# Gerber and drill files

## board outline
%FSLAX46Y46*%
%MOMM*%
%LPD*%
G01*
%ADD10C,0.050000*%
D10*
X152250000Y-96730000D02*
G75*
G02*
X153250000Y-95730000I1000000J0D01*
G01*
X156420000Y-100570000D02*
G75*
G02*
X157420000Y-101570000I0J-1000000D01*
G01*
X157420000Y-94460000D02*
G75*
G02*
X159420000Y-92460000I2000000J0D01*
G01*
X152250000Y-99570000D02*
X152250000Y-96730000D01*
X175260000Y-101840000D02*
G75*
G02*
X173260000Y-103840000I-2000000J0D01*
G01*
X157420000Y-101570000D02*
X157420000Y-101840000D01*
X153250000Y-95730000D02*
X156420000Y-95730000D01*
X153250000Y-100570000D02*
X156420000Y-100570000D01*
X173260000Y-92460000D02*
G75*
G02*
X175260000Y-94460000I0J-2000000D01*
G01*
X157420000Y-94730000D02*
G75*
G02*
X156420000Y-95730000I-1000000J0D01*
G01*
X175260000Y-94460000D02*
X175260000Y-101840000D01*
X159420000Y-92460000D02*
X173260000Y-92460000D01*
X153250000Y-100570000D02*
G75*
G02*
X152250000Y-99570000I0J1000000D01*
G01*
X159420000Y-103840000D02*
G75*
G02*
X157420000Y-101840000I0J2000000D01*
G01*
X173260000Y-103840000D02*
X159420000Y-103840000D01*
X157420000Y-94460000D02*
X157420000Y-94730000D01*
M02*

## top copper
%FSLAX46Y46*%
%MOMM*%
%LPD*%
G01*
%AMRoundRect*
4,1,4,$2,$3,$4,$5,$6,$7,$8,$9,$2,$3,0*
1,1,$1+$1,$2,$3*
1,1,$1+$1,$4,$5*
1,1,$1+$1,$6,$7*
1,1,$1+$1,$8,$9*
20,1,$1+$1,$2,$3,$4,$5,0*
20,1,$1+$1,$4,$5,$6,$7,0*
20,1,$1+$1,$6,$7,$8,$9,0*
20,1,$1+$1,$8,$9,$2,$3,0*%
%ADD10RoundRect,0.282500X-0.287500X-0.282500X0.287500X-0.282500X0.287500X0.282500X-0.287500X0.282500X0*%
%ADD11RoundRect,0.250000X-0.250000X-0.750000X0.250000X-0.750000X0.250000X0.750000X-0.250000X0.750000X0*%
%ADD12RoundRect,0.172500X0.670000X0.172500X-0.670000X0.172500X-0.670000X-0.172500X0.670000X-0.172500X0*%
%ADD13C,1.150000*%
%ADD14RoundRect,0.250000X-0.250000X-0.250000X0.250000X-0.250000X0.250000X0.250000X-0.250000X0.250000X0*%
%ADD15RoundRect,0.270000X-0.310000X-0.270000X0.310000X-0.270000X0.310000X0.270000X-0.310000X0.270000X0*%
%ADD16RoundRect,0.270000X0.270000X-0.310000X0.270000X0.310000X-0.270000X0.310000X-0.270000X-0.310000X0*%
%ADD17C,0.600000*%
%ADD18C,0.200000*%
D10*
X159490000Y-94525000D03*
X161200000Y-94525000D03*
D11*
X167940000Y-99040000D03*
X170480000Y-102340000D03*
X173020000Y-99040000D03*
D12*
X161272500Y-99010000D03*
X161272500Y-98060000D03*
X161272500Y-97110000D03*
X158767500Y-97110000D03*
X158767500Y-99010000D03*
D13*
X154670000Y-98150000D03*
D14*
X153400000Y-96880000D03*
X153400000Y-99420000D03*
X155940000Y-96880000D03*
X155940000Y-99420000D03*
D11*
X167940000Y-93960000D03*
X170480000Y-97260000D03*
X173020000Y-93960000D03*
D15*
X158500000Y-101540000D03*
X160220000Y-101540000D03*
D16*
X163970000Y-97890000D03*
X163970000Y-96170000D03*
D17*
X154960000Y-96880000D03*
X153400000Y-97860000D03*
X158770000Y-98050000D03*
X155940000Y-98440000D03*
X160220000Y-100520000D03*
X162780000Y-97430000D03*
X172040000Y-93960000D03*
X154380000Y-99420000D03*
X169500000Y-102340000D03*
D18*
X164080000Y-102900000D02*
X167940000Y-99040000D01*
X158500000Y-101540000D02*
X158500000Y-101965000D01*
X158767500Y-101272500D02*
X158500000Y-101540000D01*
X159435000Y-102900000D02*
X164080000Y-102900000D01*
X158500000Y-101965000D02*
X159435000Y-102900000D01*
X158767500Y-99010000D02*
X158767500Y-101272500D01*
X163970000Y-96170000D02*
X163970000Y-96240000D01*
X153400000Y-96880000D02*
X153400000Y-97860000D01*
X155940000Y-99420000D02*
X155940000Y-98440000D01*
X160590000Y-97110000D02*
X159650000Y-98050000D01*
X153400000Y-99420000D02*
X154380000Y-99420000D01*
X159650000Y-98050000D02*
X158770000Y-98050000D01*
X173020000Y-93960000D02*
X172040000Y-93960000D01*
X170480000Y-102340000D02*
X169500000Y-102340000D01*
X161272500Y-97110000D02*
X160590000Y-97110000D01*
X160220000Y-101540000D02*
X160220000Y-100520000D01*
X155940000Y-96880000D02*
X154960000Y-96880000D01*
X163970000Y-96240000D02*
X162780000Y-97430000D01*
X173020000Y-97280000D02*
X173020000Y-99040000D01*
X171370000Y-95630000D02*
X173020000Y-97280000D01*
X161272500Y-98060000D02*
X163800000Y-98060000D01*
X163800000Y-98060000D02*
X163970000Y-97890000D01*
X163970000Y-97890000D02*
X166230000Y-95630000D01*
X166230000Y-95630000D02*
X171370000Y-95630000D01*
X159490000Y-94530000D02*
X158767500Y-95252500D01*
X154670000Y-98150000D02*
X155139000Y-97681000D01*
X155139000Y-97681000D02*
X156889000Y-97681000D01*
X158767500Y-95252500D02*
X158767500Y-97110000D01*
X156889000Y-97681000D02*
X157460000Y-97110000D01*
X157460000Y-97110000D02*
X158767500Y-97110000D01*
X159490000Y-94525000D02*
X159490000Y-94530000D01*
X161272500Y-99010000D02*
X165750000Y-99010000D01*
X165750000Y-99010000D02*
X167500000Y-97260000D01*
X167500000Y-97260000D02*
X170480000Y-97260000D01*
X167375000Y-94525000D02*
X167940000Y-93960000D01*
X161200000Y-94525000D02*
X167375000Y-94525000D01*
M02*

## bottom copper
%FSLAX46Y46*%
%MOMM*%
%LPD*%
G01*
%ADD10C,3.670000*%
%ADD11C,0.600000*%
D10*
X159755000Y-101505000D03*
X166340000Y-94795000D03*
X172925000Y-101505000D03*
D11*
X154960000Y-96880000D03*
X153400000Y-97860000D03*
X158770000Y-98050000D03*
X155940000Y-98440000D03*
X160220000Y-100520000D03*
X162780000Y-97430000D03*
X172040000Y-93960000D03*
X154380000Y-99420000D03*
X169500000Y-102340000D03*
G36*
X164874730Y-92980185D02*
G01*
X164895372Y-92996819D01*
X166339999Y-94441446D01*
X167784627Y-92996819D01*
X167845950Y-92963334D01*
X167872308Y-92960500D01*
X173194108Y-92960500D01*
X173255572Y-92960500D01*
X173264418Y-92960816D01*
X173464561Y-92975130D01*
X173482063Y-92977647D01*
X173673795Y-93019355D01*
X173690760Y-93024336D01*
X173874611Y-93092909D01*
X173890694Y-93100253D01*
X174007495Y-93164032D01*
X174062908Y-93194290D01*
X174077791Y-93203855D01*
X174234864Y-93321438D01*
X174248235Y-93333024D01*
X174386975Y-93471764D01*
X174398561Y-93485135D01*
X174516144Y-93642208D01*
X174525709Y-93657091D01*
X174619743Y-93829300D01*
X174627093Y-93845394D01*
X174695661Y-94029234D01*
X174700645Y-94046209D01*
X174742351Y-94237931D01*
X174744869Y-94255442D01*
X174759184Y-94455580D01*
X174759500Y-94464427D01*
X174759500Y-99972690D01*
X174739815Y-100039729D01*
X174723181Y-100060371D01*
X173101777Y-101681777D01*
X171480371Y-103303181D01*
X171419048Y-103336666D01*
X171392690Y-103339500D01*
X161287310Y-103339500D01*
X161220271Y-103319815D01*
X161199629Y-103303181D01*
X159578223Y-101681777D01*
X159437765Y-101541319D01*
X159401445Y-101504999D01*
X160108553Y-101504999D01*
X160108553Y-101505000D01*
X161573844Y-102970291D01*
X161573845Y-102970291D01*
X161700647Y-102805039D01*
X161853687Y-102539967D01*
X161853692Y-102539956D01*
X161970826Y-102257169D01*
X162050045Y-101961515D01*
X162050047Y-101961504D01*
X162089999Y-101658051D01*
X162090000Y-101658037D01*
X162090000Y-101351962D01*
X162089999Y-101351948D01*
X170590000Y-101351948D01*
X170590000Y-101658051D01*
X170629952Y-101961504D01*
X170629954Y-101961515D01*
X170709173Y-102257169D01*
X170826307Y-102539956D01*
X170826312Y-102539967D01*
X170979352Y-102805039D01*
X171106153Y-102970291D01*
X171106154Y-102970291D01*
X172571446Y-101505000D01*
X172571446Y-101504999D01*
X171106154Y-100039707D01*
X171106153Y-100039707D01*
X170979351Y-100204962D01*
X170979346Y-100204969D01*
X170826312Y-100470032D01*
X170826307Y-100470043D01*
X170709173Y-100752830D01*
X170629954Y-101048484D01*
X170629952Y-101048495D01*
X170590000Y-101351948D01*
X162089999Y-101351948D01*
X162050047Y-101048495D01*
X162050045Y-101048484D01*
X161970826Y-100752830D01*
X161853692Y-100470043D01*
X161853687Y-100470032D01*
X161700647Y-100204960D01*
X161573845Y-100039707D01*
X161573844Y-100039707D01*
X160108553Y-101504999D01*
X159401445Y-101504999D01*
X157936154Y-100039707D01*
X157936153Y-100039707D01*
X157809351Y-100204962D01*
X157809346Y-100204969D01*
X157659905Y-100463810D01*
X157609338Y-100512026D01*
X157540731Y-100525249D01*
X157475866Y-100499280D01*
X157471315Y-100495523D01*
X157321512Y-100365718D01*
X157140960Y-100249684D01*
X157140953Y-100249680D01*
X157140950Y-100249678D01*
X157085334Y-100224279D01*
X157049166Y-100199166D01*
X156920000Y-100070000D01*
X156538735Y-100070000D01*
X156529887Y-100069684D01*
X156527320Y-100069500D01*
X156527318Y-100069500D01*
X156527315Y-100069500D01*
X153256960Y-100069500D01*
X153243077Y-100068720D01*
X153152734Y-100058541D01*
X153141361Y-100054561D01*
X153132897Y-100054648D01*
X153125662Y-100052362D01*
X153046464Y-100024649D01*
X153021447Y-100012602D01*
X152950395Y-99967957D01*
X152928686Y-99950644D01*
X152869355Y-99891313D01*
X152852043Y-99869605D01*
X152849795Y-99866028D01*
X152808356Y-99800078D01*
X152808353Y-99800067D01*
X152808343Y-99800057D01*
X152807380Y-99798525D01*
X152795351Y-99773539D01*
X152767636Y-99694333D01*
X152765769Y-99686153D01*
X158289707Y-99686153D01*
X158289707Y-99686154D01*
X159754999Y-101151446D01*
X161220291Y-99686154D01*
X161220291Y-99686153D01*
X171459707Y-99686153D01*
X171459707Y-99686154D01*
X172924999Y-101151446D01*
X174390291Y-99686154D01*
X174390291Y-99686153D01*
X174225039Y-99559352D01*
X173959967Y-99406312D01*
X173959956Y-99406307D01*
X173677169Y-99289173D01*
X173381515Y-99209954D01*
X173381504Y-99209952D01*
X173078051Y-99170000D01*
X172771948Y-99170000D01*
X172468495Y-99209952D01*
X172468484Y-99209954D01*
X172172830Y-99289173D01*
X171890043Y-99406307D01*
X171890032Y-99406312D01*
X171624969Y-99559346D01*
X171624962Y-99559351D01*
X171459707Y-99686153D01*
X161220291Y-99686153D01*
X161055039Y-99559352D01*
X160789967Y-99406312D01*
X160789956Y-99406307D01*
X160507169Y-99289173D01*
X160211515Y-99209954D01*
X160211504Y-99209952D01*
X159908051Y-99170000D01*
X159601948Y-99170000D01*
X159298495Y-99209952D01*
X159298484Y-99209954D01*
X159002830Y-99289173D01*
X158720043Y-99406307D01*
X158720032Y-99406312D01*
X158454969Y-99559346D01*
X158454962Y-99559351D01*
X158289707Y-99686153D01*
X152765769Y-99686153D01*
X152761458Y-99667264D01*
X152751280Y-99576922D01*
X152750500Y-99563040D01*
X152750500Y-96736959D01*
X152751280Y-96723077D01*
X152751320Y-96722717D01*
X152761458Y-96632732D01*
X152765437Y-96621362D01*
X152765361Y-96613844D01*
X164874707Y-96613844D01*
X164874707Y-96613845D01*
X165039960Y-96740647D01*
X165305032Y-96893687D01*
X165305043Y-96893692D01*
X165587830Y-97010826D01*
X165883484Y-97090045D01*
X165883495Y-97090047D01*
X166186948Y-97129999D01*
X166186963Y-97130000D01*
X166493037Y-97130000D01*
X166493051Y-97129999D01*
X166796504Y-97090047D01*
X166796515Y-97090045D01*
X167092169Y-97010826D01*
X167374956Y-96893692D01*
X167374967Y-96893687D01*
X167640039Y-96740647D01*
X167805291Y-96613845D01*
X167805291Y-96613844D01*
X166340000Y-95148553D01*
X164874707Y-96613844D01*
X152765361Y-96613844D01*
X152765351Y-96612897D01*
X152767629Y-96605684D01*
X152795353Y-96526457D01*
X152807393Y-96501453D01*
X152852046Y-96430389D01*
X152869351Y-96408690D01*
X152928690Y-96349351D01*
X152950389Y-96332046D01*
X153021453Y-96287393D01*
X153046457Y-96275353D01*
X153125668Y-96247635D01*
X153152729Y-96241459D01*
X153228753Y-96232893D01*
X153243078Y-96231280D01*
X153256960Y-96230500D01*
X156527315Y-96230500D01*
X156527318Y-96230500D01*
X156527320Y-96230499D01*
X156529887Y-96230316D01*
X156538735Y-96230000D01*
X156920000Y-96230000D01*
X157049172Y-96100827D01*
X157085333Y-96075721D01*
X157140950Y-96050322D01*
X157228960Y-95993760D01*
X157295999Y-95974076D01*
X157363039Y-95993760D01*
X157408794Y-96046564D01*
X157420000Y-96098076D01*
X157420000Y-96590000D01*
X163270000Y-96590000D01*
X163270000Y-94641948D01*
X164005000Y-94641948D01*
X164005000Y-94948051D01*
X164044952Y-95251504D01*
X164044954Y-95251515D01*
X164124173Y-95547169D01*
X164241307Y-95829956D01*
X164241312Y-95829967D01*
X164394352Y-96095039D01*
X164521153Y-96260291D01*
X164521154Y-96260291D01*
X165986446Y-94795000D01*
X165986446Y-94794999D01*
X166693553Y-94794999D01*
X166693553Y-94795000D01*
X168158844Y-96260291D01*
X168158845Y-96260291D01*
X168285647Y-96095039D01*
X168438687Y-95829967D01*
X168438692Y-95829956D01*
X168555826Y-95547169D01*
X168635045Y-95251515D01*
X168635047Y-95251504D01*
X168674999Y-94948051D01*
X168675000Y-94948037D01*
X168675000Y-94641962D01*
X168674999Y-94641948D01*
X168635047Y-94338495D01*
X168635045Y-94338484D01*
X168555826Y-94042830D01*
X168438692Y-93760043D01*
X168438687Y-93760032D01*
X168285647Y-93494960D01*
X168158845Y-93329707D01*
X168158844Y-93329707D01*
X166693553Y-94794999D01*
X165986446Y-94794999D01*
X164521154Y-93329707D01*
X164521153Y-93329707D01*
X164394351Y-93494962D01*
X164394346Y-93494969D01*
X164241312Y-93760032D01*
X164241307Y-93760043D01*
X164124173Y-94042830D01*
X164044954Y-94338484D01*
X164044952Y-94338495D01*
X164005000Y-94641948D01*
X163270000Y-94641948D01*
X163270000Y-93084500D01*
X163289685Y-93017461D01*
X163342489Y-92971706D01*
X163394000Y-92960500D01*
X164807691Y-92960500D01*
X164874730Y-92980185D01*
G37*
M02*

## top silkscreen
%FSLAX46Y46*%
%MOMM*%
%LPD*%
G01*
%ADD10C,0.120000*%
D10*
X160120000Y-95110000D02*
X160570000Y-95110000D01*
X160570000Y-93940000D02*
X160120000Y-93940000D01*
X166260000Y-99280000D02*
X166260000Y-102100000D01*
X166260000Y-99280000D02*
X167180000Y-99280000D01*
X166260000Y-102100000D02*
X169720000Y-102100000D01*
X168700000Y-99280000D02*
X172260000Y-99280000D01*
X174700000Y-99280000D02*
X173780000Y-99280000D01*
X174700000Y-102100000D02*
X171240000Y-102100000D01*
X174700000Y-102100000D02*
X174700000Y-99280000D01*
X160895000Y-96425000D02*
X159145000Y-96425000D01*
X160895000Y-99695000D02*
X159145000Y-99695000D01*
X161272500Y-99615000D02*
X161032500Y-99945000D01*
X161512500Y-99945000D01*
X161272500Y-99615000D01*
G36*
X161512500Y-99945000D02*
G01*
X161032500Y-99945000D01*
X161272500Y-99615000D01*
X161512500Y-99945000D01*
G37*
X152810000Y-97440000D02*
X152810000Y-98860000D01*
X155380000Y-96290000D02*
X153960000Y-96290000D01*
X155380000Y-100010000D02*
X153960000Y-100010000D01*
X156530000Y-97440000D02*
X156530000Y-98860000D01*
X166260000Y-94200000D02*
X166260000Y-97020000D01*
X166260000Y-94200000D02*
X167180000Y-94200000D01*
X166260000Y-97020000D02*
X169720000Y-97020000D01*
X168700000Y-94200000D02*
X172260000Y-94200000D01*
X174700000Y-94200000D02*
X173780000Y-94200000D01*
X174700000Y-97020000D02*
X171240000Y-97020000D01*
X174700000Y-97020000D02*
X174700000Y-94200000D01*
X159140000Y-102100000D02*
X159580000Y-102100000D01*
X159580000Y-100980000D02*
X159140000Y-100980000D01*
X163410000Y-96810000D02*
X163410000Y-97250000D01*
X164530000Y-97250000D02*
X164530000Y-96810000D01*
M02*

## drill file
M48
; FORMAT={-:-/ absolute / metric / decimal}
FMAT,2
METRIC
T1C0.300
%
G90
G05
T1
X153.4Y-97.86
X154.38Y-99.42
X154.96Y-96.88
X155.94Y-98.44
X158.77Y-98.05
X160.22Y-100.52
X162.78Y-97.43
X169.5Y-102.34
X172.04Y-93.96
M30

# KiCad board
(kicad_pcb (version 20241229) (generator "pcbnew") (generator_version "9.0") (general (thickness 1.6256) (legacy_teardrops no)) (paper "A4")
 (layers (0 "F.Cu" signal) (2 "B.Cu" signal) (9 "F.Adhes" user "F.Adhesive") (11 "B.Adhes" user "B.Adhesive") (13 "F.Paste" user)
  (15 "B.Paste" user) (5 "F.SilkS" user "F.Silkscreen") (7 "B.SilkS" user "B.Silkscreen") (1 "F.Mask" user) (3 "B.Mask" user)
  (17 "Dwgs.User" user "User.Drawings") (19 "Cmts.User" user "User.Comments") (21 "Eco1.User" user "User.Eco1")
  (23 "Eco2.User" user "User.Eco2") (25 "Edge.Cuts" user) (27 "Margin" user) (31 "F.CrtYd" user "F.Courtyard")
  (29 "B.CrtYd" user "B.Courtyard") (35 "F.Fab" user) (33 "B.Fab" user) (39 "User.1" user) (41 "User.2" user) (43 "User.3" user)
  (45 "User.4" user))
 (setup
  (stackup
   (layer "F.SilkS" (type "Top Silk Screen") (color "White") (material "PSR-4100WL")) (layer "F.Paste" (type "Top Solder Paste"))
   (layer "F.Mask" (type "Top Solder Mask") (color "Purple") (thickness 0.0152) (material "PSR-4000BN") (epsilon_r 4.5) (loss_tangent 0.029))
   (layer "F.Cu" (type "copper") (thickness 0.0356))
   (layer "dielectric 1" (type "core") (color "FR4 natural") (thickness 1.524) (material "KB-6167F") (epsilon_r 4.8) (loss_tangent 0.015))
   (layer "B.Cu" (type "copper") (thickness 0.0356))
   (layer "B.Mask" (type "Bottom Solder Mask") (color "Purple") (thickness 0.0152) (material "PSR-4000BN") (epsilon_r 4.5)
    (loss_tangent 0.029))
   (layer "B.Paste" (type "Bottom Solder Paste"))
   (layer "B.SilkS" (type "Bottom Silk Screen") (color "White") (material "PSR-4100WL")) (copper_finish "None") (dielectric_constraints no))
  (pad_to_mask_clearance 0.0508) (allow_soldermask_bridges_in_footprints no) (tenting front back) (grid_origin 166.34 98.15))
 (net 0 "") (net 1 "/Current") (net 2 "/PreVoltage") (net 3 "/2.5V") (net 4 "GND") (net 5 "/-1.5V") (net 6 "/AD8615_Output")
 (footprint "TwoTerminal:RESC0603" (layer "F.Cu") (at 160.345 94.525)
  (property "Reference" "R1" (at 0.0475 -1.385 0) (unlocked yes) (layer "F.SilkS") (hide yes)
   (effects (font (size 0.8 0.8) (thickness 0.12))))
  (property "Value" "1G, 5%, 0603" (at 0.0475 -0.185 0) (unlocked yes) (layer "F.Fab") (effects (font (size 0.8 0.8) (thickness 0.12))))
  (fp_line (start -0.225 0.585) (end 0.225 0.585) (stroke (width 0.12) (type default)) (layer "F.SilkS"))
  (fp_line (start 0.225 -0.585) (end -0.225 -0.585) (stroke (width 0.12) (type default)) (layer "F.SilkS"))
  (pad "1" smd roundrect (at -0.855 0) (size 1.14 1.13) (layers "F.Cu" "F.Mask" "F.Paste") (roundrect_rratio 0.25) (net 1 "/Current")
   (thermal_bridge_angle 45))
  (pad "2" smd roundrect (at 0.855 0) (size 1.14 1.13) (layers "F.Cu" "F.Mask" "F.Paste") (roundrect_rratio 0.25) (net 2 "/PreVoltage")
   (thermal_bridge_angle 45)))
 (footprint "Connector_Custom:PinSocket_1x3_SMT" (layer "F.Cu") (at 170.48 100.69 90)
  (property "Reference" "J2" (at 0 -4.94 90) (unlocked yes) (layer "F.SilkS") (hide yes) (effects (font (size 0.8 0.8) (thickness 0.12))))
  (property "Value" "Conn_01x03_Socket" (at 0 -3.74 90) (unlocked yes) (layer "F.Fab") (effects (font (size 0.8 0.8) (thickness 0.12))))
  (fp_line (start 1.41 -4.22) (end -1.41 -4.22) (stroke (width 0.12) (type default)) (layer "F.SilkS"))
  (fp_line (start 1.41 -4.22) (end 1.41 -3.3) (stroke (width 0.12) (type default)) (layer "F.SilkS"))
  (fp_line (start -1.41 -4.22) (end -1.41 -0.76) (stroke (width 0.12) (type default)) (layer "F.SilkS"))
  (fp_line (start 1.41 -1.78) (end 1.41 1.78) (stroke (width 0.12) (type default)) (layer "F.SilkS"))
  (fp_line (start 1.41 4.22) (end 1.41 3.3) (stroke (width 0.12) (type default)) (layer "F.SilkS"))
  (fp_line (start -1.41 4.22) (end -1.41 0.76) (stroke (width 0.12) (type default)) (layer "F.SilkS"))
  (fp_line (start -1.41 4.22) (end 1.41 4.22) (stroke (width 0.12) (type default)) (layer "F.SilkS"))
  (pad "1" smd roundrect (at 1.65 -2.54) (size 1 2) (layers "F.Cu" "F.Mask" "F.Paste") (roundrect_rratio 0.25) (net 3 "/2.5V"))
  (pad "2" smd roundrect (at -1.65 0) (size 1 2) (layers "F.Cu" "F.Mask" "F.Paste") (roundrect_rratio 0.25) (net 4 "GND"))
  (pad "3" smd roundrect (at 1.65 2.54) (size 1 2) (layers "F.Cu" "F.Mask" "F.Paste") (roundrect_rratio 0.25) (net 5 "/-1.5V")))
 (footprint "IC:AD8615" (layer "F.Cu") (at 160.02 98.06 180)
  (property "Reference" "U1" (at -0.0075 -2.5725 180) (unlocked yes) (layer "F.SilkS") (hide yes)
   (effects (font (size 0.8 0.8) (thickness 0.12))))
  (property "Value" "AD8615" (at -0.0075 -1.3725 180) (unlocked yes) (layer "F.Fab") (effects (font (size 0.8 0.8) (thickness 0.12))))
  (fp_line (start -0.875 1.635) (end 0.875 1.635) (stroke (width 0.12) (type default)) (layer "F.SilkS"))
  (fp_line (start -0.875 -1.635) (end 0.875 -1.635) (stroke (width 0.12) (type default)) (layer "F.SilkS"))
  (fp_poly
   (pts (xy -1.2525 -1.555) (xy -1.0125 -1.885) (xy -1.4925 -1.885)) (stroke (width 0.12) (type solid)) (fill yes) (layer "F.SilkS"))
  (pad "1" smd roundrect (at -1.2525 -0.95 180) (size 1.685 0.69) (layers "F.Cu" "F.Mask" "F.Paste") (roundrect_rratio 0.25)
   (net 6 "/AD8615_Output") (thermal_bridge_angle 45))
  (pad "2" smd roundrect (at -1.2525 0 180) (size 1.685 0.69) (layers "F.Cu" "F.Mask" "F.Paste") (roundrect_rratio 0.25) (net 5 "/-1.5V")
   (thermal_bridge_angle 45))
  (pad "3" smd roundrect (at -1.2525 0.95 180) (size 1.685 0.69) (layers "F.Cu" "F.Mask" "F.Paste") (roundrect_rratio 0.25) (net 4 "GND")
   (thermal_bridge_angle 45))
  (pad "4" smd roundrect (at 1.2525 0.95 180) (size 1.685 0.69) (layers "F.Cu" "F.Mask" "F.Paste") (roundrect_rratio 0.25)
   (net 1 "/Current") (thermal_bridge_angle 45))
  (pad "5" smd roundrect (at 1.2525 -0.95 180) (size 1.685 0.69) (layers "F.Cu" "F.Mask" "F.Paste") (roundrect_rratio 0.25) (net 3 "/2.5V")
   (thermal_bridge_angle 45)))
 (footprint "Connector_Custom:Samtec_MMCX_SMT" (layer "F.Cu") (at 154.67 98.15)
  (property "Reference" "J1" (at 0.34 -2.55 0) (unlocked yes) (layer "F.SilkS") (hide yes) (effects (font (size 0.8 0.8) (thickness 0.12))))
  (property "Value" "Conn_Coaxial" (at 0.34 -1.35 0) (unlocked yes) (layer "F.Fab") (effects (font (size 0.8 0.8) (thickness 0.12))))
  (fp_line (start -1.86 -0.71) (end -1.86 0.71) (stroke (width 0.12) (type default)) (layer "F.SilkS"))
  (fp_line (start 0.71 -1.86) (end -0.71 -1.86) (stroke (width 0.12) (type default)) (layer "F.SilkS"))
  (fp_line (start 0.71 1.86) (end -0.71 1.86) (stroke (width 0.12) (type default)) (layer "F.SilkS"))
  (fp_line (start 1.86 -0.71) (end 1.86 0.71) (stroke (width 0.12) (type default)) (layer "F.SilkS"))
  (pad "1" smd circle (at 0 0) (size 1.15 1.15) (layers "F.Cu" "F.Mask" "F.Paste") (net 1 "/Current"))
  (pad "2" smd roundrect (at -1.27 -1.27) (size 1 1) (layers "F.Cu" "F.Mask" "F.Paste") (roundrect_rratio 0.25) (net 4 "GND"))
  (pad "2" smd roundrect (at -1.27 1.27) (size 1 1) (layers "F.Cu" "F.Mask" "F.Paste") (roundrect_rratio 0.25) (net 4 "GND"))
  (pad "2" smd roundrect (at 1.27 -1.27) (size 1 1) (layers "F.Cu" "F.Mask" "F.Paste") (roundrect_rratio 0.25) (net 4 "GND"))
  (pad "2" smd roundrect (at 1.27 1.27) (size 1 1) (layers "F.Cu" "F.Mask" "F.Paste") (roundrect_rratio 0.25) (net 4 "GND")))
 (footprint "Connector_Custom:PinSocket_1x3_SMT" (layer "F.Cu") (at 170.48 95.61 90)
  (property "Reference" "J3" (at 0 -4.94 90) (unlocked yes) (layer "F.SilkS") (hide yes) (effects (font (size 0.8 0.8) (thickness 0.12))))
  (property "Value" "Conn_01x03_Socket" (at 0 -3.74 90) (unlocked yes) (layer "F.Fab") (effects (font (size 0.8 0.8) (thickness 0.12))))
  (fp_line (start 1.41 -4.22) (end -1.41 -4.22) (stroke (width 0.12) (type default)) (layer "F.SilkS"))
  (fp_line (start 1.41 -4.22) (end 1.41 -3.3) (stroke (width 0.12) (type default)) (layer "F.SilkS"))
  (fp_line (start -1.41 -4.22) (end -1.41 -0.76) (stroke (width 0.12) (type default)) (layer "F.SilkS"))
  (fp_line (start 1.41 -1.78) (end 1.41 1.78) (stroke (width 0.12) (type default)) (layer "F.SilkS"))
  (fp_line (start 1.41 4.22) (end 1.41 3.3) (stroke (width 0.12) (type default)) (layer "F.SilkS"))
  (fp_line (start -1.41 4.22) (end -1.41 0.76) (stroke (width 0.12) (type default)) (layer "F.SilkS"))
  (fp_line (start -1.41 4.22) (end 1.41 4.22) (stroke (width 0.12) (type default)) (layer "F.SilkS"))
  (pad "1" smd roundrect (at 1.65 -2.54) (size 1 2) (layers "F.Cu" "F.Mask" "F.Paste") (roundrect_rratio 0.25) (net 2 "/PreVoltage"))
  (pad "2" smd roundrect (at -1.65 0) (size 1 2) (layers "F.Cu" "F.Mask" "F.Paste") (roundrect_rratio 0.25) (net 6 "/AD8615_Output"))
  (pad "3" smd roundrect (at 1.65 2.54) (size 1 2) (layers "F.Cu" "F.Mask" "F.Paste") (roundrect_rratio 0.25) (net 4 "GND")))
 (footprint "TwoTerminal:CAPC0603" (layer "F.Cu") (at 159.36 101.54)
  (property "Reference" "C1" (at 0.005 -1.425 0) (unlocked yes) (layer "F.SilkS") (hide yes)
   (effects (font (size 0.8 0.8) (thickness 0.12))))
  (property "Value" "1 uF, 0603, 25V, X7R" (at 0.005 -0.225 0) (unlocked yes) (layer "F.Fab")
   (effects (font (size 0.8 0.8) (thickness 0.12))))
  (fp_line (start -0.22 0.56) (end 0.22 0.56) (stroke (width 0.12) (type default)) (layer "F.SilkS"))
  (fp_line (start 0.22 -0.56) (end -0.22 -0.56) (stroke (width 0.12) (type default)) (layer "F.SilkS"))
  (pad "1" smd roundrect (at -0.86 0) (size 1.16 1.08) (layers "F.Cu" "F.Mask" "F.Paste") (roundrect_rratio 0.25) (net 3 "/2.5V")
   (thermal_bridge_angle 45))
  (pad "2" smd roundrect (at 0.86 0) (size 1.16 1.08) (layers "F.Cu" "F.Mask" "F.Paste") (roundrect_rratio 0.25) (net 4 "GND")
   (thermal_bridge_angle 45)))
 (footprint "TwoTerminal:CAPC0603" (layer "F.Cu") (at 163.97 97.03 90)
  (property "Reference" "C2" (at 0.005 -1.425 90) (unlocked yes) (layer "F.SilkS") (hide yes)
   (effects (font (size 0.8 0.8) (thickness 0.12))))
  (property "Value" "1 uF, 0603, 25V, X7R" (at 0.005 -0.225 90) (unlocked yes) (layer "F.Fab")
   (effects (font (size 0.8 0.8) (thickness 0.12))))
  (fp_line (start 0.22 -0.56) (end -0.22 -0.56) (stroke (width 0.12) (type default)) (layer "F.SilkS"))
  (fp_line (start -0.22 0.56) (end 0.22 0.56) (stroke (width 0.12) (type default)) (layer "F.SilkS"))
  (pad "1" smd roundrect (at -0.86 0 90) (size 1.16 1.08) (layers "F.Cu" "F.Mask" "F.Paste") (roundrect_rratio 0.25) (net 5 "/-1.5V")
   (thermal_bridge_angle 45))
  (pad "2" smd roundrect (at 0.86 0 90) (size 1.16 1.08) (layers "F.Cu" "F.Mask" "F.Paste") (roundrect_rratio 0.25) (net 4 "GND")
   (thermal_bridge_angle 45)))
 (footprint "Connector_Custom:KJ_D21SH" (layer "B.Cu") (at 159.755 101.505)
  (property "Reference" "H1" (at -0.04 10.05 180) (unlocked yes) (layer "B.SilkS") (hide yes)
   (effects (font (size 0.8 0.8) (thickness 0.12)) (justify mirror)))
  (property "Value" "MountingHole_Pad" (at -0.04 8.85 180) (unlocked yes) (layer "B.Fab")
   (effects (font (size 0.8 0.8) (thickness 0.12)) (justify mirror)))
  (pad "1" smd circle (at 0 0) (size 3.67 3.67) (layers "B.Cu" "B.Mask") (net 4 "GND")))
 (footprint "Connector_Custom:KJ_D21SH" (layer "B.Cu") (at 166.34 94.795)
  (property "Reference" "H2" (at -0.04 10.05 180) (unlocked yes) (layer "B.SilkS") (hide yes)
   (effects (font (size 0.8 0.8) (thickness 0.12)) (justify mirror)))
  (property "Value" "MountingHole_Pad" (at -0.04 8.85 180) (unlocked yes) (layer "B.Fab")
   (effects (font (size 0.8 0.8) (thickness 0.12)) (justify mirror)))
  (pad "1" smd circle (at 0 0) (size 3.67 3.67) (layers "B.Cu" "B.Mask") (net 4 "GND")))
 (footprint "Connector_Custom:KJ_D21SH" (layer "B.Cu") (at 172.925 101.505)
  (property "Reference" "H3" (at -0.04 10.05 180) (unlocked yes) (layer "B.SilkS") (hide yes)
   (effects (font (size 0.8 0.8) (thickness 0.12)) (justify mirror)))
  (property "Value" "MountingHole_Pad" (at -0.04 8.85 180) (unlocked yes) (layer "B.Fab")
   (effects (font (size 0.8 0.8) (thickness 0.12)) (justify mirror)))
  (pad "1" smd circle (at 0 0) (size 3.67 3.67) (layers "B.Cu" "B.Mask") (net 4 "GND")))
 (gr_arc (start 152.25 96.73) (mid 152.542893 96.022893) (end 153.25 95.73) (stroke (width 0.05) (type default)) (layer "Edge.Cuts"))
 (gr_arc (start 156.42 100.57) (mid 157.127107 100.862893) (end 157.42 101.57) (stroke (width 0.05) (type default)) (layer "Edge.Cuts"))
 (gr_arc (start 157.42 94.46) (mid 158.005786 93.045786) (end 159.42 92.46) (stroke (width 0.05) (type default)) (layer "Edge.Cuts"))
 (gr_line (start 152.25 99.57) (end 152.25 96.73) (stroke (width 0.05) (type default)) (layer "Edge.Cuts"))
 (gr_arc (start 175.26 101.84) (mid 174.674214 103.254214) (end 173.26 103.84) (stroke (width 0.05) (type default)) (layer "Edge.Cuts"))
 (gr_line (start 157.42 101.57) (end 157.42 101.84) (stroke (width 0.05) (type default)) (layer "Edge.Cuts"))
 (gr_line (start 153.25 95.73) (end 156.42 95.73) (stroke (width 0.05) (type default)) (layer "Edge.Cuts"))
 (gr_line (start 153.25 100.57) (end 156.42 100.57) (stroke (width 0.05) (type default)) (layer "Edge.Cuts"))
 (gr_arc (start 173.26 92.46) (mid 174.674214 93.045786) (end 175.26 94.46) (stroke (width 0.05) (type default)) (layer "Edge.Cuts"))
 (gr_arc (start 157.42 94.73) (mid 157.127107 95.437107) (end 156.42 95.73) (stroke (width 0.05) (type default)) (layer "Edge.Cuts"))
 (gr_line (start 175.26 94.46) (end 175.26 101.84) (stroke (width 0.05) (type default)) (layer "Edge.Cuts"))
 (gr_line (start 159.42 92.46) (end 173.26 92.46) (stroke (width 0.05) (type default)) (layer "Edge.Cuts"))
 (gr_arc (start 153.25 100.57) (mid 152.542893 100.277107) (end 152.25 99.57) (stroke (width 0.05) (type default)) (layer "Edge.Cuts"))
 (gr_arc (start 159.42 103.84) (mid 158.005786 103.254214) (end 157.42 101.84) (stroke (width 0.05) (type default)) (layer "Edge.Cuts"))
 (gr_line (start 173.26 103.84) (end 159.42 103.84) (stroke (width 0.05) (type default)) (layer "Edge.Cuts"))
 (gr_line (start 157.42 94.46) (end 157.42 94.73) (stroke (width 0.05) (type default)) (layer "Edge.Cuts"))
 (segment (start 164.08 102.9) (end 167.94 99.04) (width 0.2) (layer "F.Cu") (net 3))
 (segment (start 158.5 101.54) (end 158.5 101.965) (width 0.2) (layer "F.Cu") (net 3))
 (segment (start 158.7675 101.2725) (end 158.5 101.54) (width 0.2) (layer "F.Cu") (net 3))
 (segment (start 159.435 102.9) (end 164.08 102.9) (width 0.2) (layer "F.Cu") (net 3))
 (segment (start 158.5 101.965) (end 159.435 102.9) (width 0.2) (layer "F.Cu") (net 3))
 (segment (start 158.7675 99.01) (end 158.7675 101.2725) (width 0.2) (layer "F.Cu") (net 3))
 (segment (start 163.97 96.17) (end 163.97 96.24) (width 0.2) (layer "F.Cu") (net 4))
 (segment (start 153.4 96.88) (end 153.4 97.86) (width 0.2) (layer "F.Cu") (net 4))
 (segment (start 155.94 99.42) (end 155.94 98.44) (width 0.2) (layer "F.Cu") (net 4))
 (segment (start 160.59 97.11) (end 159.65 98.05) (width 0.2) (layer "F.Cu") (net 4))
 (segment (start 153.4 99.42) (end 154.38 99.42) (width 0.2) (layer "F.Cu") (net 4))
 (segment (start 159.65 98.05) (end 158.77 98.05) (width 0.2) (layer "F.Cu") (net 4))
 (segment (start 173.02 93.96) (end 172.04 93.96) (width 0.2) (layer "F.Cu") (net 4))
 (segment (start 170.48 102.34) (end 169.5 102.34) (width 0.2) (layer "F.Cu") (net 4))
 (segment (start 161.2725 97.11) (end 160.59 97.11) (width 0.2) (layer "F.Cu") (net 4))
 (segment (start 160.22 101.54) (end 160.22 100.52) (width 0.2) (layer "F.Cu") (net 4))
 (segment (start 155.94 96.88) (end 154.96 96.88) (width 0.2) (layer "F.Cu") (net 4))
 (segment (start 163.97 96.24) (end 162.78 97.43) (width 0.2) (layer "F.Cu") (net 4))
 (via (at 154.96 96.88) (size 0.6) (drill 0.3) (layers "F.Cu" "B.Cu") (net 4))
 (via (at 153.4 97.86) (size 0.6) (drill 0.3) (layers "F.Cu" "B.Cu") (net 4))
 (via (at 158.77 98.05) (size 0.6) (drill 0.3) (layers "F.Cu" "B.Cu") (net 4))
 (via (at 155.94 98.44) (size 0.6) (drill 0.3) (layers "F.Cu" "B.Cu") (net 4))
 (via (at 160.22 100.52) (size 0.6) (drill 0.3) (layers "F.Cu" "B.Cu") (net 4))
 (via (at 162.78 97.43) (size 0.6) (drill 0.3) (layers "F.Cu" "B.Cu") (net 4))
 (via (at 172.04 93.96) (size 0.6) (drill 0.3) (layers "F.Cu" "B.Cu") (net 4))
 (via (at 154.38 99.42) (size 0.6) (drill 0.3) (layers "F.Cu" "B.Cu") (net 4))
 (via (at 169.5 102.34) (size 0.6) (drill 0.3) (layers "F.Cu" "B.Cu") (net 4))
 (segment (start 173.02 97.28) (end 173.02 99.04) (width 0.2) (layer "F.Cu") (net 5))
 (segment (start 171.37 95.63) (end 173.02 97.28) (width 0.2) (layer "F.Cu") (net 5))
 (segment (start 161.2725 98.06) (end 163.8 98.06) (width 0.2) (layer "F.Cu") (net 5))
 (segment (start 163.8 98.06) (end 163.97 97.89) (width 0.2) (layer "F.Cu") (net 5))
 (segment (start 163.97 97.89) (end 166.23 95.63) (width 0.2) (layer "F.Cu") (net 5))
 (segment (start 166.23 95.63) (end 171.37 95.63) (width 0.2) (layer "F.Cu") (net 5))
 (segment (start 159.49 94.53) (end 158.7675 95.2525) (width 0.2) (layer "F.Cu") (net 1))
 (segment (start 154.67 98.15) (end 155.139 97.681) (width 0.2) (layer "F.Cu") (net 1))
 (segment (start 155.139 97.681) (end 156.889 97.681) (width 0.2) (layer "F.Cu") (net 1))
 (segment (start 158.7675 95.2525) (end 158.7675 97.11) (width 0.2) (layer "F.Cu") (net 1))
 (segment (start 156.889 97.681) (end 157.46 97.11) (width 0.2) (layer "F.Cu") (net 1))
 (segment (start 157.46 97.11) (end 158.7675 97.11) (width 0.2) (layer "F.Cu") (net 1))
 (segment (start 159.49 94.525) (end 159.49 94.53) (width 0.2) (layer "F.Cu") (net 1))
 (segment (start 161.2725 99.01) (end 165.75 99.01) (width 0.2) (layer "F.Cu") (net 6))
 (segment (start 165.75 99.01) (end 167.5 97.26) (width 0.2) (layer "F.Cu") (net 6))
 (segment (start 167.5 97.26) (end 170.48 97.26) (width 0.2) (layer "F.Cu") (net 6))
 (segment (start 167.375 94.525) (end 167.94 93.96) (width 0.2) (layer "F.Cu") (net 2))
 (segment (start 161.2 94.525) (end 167.375 94.525) (width 0.2) (layer "F.Cu") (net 2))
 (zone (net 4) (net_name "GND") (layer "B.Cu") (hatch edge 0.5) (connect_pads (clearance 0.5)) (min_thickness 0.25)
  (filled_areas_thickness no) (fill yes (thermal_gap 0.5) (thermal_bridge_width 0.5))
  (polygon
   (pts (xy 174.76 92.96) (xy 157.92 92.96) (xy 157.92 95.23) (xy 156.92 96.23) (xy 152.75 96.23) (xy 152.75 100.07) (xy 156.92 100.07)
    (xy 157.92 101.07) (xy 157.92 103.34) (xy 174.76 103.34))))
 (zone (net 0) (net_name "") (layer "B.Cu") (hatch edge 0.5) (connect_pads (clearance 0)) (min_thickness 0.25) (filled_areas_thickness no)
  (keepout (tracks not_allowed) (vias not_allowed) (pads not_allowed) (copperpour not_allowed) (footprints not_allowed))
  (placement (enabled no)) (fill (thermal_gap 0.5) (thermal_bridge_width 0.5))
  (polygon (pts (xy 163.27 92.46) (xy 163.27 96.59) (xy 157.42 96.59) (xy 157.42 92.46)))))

